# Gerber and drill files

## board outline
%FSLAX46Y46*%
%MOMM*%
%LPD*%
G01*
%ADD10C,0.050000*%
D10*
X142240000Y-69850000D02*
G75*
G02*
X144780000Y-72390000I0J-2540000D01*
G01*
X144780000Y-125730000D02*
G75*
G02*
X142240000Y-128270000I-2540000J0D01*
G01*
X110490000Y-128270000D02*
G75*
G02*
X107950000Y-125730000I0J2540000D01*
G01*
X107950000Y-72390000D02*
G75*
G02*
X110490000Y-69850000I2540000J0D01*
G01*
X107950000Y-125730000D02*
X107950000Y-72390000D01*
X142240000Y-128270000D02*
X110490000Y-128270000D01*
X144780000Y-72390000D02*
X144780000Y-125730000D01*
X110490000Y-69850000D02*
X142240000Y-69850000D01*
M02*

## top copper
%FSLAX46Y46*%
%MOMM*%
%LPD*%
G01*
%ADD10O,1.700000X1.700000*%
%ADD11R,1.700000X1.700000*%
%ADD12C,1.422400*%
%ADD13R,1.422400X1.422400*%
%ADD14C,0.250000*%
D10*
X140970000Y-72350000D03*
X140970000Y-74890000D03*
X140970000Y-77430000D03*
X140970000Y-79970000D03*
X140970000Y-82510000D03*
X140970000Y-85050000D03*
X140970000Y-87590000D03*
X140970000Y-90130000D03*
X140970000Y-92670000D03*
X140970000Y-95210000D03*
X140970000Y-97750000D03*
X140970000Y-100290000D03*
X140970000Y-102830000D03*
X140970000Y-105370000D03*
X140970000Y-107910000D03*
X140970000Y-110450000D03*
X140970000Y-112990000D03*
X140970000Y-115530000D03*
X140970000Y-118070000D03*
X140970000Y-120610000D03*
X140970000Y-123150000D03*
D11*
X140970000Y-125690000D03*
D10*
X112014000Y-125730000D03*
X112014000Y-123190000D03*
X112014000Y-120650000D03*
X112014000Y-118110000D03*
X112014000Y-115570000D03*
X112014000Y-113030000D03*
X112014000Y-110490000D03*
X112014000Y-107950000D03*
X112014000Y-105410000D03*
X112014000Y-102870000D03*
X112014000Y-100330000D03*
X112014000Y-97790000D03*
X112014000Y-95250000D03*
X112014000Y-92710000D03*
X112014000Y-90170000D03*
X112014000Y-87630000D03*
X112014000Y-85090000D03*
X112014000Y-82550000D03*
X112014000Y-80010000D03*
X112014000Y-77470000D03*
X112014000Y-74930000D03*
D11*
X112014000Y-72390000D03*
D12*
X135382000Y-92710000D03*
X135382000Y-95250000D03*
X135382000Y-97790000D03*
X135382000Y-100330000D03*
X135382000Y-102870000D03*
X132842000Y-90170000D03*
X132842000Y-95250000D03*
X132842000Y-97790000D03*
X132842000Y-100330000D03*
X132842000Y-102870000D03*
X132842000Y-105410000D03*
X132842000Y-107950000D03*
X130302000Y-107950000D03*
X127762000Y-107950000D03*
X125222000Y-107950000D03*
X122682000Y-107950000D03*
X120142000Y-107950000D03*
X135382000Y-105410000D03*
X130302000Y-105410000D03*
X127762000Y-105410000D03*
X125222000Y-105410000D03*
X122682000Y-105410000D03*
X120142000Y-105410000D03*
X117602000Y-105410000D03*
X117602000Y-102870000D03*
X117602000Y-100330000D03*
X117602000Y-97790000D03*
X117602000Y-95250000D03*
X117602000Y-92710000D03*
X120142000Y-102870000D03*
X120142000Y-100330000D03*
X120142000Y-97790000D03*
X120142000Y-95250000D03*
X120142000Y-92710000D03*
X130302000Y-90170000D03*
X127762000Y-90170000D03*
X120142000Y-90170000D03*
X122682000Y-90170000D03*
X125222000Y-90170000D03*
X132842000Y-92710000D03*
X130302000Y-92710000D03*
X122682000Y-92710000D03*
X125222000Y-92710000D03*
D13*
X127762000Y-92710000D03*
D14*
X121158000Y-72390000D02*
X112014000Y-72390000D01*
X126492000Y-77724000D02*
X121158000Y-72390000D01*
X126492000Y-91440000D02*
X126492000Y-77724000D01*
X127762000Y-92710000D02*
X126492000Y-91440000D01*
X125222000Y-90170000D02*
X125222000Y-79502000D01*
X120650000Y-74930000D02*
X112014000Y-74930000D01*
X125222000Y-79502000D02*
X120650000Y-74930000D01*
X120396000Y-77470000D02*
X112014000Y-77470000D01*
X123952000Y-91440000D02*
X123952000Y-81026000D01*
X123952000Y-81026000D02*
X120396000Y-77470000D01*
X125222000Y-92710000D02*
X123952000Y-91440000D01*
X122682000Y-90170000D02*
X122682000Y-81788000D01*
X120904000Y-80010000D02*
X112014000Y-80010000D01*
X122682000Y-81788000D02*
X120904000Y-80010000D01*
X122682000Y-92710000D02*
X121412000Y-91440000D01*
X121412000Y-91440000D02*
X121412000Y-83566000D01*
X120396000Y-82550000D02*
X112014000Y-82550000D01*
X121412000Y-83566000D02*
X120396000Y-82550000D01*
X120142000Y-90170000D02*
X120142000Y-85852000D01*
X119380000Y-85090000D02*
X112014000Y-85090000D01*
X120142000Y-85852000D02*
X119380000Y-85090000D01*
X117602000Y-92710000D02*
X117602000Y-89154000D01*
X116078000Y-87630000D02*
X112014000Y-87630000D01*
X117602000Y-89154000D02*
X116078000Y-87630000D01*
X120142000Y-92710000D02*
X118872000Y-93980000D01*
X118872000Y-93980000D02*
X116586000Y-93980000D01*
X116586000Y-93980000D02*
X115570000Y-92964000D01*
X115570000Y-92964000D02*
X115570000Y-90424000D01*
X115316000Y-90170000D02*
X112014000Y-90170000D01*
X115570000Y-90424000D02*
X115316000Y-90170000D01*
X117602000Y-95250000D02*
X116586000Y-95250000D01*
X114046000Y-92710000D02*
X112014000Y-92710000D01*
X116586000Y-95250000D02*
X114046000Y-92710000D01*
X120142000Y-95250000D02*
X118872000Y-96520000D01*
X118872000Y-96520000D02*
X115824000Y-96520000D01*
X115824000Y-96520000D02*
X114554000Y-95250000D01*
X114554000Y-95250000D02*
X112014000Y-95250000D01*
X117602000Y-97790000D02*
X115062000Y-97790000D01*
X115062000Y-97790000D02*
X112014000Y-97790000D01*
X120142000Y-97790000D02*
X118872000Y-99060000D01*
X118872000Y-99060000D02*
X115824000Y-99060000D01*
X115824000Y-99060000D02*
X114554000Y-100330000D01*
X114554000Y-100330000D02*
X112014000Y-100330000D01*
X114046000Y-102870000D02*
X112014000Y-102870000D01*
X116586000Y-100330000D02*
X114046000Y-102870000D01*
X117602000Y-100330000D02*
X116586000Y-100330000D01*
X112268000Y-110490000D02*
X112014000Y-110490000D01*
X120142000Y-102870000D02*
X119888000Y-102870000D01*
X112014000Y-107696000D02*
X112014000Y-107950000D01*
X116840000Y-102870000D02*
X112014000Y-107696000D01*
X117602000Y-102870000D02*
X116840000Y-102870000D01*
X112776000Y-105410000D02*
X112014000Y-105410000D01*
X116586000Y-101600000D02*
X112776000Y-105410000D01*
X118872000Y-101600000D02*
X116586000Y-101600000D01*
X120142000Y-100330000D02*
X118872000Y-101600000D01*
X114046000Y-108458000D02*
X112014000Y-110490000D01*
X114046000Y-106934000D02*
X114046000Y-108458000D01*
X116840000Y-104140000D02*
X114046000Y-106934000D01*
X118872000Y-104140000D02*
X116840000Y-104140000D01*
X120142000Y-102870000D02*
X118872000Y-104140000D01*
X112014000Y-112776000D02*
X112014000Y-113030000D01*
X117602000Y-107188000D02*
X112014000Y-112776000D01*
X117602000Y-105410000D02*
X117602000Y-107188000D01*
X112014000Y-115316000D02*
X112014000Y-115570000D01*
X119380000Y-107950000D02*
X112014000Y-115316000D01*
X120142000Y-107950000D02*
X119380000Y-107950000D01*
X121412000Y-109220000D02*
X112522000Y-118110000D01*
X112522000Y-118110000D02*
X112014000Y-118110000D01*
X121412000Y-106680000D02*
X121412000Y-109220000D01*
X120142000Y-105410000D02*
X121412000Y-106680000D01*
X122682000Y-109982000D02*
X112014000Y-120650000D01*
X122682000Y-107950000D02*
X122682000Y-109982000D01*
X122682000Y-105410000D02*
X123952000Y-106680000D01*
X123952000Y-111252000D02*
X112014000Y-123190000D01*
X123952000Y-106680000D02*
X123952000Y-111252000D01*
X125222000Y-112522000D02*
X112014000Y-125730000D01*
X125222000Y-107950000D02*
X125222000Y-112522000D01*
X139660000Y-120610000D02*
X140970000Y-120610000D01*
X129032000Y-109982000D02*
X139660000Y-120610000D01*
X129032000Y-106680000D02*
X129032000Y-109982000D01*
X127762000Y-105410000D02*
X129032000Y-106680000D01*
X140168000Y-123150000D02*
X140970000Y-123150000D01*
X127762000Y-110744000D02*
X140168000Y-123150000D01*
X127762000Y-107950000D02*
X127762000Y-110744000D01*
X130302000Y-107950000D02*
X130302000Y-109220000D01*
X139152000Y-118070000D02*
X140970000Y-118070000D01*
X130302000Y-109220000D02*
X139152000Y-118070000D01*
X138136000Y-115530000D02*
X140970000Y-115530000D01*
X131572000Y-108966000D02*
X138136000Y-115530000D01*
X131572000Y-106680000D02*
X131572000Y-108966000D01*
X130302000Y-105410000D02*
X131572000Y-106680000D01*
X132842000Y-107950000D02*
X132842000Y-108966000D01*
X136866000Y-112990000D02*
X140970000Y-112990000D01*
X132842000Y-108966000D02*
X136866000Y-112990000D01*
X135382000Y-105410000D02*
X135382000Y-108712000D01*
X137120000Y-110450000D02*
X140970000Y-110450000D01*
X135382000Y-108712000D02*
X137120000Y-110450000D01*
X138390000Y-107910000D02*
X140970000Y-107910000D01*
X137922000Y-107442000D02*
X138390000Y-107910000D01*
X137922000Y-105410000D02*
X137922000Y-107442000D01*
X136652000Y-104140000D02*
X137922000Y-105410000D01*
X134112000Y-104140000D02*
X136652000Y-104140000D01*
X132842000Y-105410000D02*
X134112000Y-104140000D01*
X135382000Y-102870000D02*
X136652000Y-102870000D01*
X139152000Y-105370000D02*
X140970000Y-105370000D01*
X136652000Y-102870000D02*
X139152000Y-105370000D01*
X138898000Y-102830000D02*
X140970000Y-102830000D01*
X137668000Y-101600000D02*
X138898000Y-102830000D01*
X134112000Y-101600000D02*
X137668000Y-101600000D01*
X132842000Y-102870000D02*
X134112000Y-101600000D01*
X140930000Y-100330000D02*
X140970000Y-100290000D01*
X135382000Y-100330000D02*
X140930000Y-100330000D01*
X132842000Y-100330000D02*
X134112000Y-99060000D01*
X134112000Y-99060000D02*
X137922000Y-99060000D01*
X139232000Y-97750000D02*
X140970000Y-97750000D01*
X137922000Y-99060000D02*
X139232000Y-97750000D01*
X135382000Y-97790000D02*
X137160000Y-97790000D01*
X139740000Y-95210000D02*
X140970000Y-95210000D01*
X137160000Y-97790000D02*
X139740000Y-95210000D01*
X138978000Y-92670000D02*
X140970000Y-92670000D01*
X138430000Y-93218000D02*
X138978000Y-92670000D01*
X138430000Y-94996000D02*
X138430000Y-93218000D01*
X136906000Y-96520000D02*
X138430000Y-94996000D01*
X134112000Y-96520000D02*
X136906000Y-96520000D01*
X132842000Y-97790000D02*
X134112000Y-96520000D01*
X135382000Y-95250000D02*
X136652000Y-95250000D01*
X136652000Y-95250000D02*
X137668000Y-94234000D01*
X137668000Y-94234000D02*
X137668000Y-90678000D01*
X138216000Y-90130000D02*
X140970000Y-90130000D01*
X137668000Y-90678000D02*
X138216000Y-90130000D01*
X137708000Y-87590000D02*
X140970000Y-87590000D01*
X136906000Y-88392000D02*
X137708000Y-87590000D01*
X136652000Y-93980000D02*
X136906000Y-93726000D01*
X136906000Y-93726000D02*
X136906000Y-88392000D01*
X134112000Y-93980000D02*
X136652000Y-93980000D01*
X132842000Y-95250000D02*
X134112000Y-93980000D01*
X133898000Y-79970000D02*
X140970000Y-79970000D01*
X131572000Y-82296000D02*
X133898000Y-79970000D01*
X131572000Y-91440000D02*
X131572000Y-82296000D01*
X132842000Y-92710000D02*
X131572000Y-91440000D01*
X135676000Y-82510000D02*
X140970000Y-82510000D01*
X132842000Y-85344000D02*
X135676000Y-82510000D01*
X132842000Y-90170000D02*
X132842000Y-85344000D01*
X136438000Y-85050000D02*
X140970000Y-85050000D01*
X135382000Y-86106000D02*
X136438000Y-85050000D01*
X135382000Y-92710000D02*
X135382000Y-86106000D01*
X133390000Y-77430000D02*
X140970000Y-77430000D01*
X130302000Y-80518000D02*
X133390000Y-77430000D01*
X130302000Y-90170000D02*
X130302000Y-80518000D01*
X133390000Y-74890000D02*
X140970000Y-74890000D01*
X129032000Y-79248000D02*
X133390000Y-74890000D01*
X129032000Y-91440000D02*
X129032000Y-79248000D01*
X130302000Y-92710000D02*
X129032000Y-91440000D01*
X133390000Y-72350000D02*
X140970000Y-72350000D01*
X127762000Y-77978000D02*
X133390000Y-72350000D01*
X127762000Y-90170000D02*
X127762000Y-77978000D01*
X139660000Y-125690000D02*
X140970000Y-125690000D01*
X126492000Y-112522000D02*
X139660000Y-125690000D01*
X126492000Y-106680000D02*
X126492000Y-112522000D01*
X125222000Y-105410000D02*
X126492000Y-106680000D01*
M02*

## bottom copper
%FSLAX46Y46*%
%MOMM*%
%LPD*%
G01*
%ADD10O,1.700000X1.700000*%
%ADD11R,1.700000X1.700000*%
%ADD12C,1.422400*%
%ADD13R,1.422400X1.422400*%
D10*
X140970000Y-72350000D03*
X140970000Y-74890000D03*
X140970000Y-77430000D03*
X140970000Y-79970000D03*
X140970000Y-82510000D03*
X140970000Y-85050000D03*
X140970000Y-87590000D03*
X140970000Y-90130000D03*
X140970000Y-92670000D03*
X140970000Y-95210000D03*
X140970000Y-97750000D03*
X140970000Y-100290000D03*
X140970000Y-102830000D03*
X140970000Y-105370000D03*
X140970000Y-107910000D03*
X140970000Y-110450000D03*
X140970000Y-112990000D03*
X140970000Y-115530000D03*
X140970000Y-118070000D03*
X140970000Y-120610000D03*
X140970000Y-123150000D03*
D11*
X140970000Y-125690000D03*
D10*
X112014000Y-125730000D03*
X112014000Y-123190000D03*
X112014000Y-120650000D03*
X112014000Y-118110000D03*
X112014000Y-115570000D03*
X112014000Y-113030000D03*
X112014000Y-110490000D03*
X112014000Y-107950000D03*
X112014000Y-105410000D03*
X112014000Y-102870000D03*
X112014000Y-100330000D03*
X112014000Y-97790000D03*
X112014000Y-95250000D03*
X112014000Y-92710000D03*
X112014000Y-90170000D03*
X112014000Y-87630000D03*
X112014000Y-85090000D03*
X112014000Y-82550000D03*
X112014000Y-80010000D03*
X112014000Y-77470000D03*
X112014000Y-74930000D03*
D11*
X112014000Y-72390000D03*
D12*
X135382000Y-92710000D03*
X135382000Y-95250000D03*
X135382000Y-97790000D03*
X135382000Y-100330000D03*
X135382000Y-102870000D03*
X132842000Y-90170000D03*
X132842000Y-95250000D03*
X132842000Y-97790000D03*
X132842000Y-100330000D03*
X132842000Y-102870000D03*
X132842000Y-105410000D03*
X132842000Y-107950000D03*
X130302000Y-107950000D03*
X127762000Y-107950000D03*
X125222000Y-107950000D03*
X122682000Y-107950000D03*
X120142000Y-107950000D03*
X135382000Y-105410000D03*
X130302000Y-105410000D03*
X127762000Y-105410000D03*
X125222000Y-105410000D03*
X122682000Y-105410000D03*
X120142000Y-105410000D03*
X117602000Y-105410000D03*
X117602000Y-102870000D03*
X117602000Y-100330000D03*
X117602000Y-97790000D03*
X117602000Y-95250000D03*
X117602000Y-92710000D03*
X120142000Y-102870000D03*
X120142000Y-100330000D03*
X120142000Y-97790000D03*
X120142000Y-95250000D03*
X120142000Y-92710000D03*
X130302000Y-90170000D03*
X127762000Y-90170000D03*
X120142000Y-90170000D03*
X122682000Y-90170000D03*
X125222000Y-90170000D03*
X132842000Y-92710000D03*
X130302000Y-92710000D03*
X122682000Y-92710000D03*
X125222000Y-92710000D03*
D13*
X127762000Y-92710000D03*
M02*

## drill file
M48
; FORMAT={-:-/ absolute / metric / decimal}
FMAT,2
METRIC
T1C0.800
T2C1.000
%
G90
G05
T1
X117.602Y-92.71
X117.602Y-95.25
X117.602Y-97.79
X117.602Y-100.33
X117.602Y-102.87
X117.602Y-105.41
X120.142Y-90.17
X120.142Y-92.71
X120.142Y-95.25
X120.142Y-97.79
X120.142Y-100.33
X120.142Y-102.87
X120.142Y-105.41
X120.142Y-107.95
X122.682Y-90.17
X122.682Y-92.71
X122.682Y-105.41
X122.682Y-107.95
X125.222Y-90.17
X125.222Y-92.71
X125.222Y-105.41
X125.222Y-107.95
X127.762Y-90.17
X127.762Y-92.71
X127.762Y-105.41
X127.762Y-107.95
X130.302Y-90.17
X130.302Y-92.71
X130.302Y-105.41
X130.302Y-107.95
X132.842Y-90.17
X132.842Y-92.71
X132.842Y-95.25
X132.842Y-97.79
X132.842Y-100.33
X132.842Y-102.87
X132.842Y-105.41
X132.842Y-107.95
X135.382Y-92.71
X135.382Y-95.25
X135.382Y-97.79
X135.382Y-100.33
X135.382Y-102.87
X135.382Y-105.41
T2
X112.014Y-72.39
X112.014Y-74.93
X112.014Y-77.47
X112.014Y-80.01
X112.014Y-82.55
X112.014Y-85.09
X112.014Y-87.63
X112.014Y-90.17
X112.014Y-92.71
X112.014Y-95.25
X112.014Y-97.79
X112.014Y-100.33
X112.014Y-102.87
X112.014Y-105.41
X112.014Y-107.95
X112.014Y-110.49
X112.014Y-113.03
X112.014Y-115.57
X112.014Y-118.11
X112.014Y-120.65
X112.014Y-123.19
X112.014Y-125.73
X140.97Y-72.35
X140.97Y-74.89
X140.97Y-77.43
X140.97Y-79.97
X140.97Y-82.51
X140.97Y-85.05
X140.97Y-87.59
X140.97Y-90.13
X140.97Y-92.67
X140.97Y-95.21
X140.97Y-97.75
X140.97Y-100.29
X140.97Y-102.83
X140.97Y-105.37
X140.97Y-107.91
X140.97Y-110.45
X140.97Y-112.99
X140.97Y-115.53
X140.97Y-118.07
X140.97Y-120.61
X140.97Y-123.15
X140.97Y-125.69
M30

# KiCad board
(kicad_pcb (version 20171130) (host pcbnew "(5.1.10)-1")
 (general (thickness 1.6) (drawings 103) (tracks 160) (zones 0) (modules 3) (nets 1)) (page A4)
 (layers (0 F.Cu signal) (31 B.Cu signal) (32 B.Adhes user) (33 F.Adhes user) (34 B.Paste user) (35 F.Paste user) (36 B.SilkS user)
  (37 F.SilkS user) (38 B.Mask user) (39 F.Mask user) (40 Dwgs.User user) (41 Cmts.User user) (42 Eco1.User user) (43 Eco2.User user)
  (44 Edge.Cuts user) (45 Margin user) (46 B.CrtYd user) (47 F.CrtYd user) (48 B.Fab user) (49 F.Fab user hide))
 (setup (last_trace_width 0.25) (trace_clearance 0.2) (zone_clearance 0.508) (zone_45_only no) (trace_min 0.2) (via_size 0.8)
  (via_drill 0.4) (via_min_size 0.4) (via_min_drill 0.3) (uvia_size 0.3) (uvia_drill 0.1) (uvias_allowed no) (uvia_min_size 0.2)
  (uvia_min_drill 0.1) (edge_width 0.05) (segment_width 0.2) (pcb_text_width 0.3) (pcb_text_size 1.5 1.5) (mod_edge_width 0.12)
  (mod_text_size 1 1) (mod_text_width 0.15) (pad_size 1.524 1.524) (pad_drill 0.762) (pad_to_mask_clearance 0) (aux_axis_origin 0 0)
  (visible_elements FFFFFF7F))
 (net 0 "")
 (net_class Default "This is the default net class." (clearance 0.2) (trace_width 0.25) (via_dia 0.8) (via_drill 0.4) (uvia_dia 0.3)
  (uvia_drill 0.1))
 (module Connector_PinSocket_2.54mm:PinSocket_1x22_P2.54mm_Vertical (layer F.Cu) (at 140.97 125.69 180)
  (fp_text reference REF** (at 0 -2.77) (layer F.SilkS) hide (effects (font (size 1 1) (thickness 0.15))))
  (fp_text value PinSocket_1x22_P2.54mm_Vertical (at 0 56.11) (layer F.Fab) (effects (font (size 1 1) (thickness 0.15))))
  (pad 22 thru_hole oval (at 0 53.34 180) (size 1.7 1.7) (drill 1) (layers *.Cu *.Mask))
  (pad 21 thru_hole oval (at 0 50.8 180) (size 1.7 1.7) (drill 1) (layers *.Cu *.Mask))
  (pad 20 thru_hole oval (at 0 48.26 180) (size 1.7 1.7) (drill 1) (layers *.Cu *.Mask))
  (pad 19 thru_hole oval (at 0 45.72 180) (size 1.7 1.7) (drill 1) (layers *.Cu *.Mask))
  (pad 18 thru_hole oval (at 0 43.18 180) (size 1.7 1.7) (drill 1) (layers *.Cu *.Mask))
  (pad 17 thru_hole oval (at 0 40.64 180) (size 1.7 1.7) (drill 1) (layers *.Cu *.Mask))
  (pad 16 thru_hole oval (at 0 38.1 180) (size 1.7 1.7) (drill 1) (layers *.Cu *.Mask))
  (pad 15 thru_hole oval (at 0 35.56 180) (size 1.7 1.7) (drill 1) (layers *.Cu *.Mask))
  (pad 14 thru_hole oval (at 0 33.02 180) (size 1.7 1.7) (drill 1) (layers *.Cu *.Mask))
  (pad 13 thru_hole oval (at 0 30.48 180) (size 1.7 1.7) (drill 1) (layers *.Cu *.Mask))
  (pad 12 thru_hole oval (at 0 27.94 180) (size 1.7 1.7) (drill 1) (layers *.Cu *.Mask))
  (pad 11 thru_hole oval (at 0 25.4 180) (size 1.7 1.7) (drill 1) (layers *.Cu *.Mask))
  (pad 10 thru_hole oval (at 0 22.86 180) (size 1.7 1.7) (drill 1) (layers *.Cu *.Mask))
  (pad 9 thru_hole oval (at 0 20.32 180) (size 1.7 1.7) (drill 1) (layers *.Cu *.Mask))
  (pad 8 thru_hole oval (at 0 17.78 180) (size 1.7 1.7) (drill 1) (layers *.Cu *.Mask))
  (pad 7 thru_hole oval (at 0 15.24 180) (size 1.7 1.7) (drill 1) (layers *.Cu *.Mask))
  (pad 6 thru_hole oval (at 0 12.7 180) (size 1.7 1.7) (drill 1) (layers *.Cu *.Mask))
  (pad 5 thru_hole oval (at 0 10.16 180) (size 1.7 1.7) (drill 1) (layers *.Cu *.Mask))
  (pad 4 thru_hole oval (at 0 7.62 180) (size 1.7 1.7) (drill 1) (layers *.Cu *.Mask))
  (pad 3 thru_hole oval (at 0 5.08 180) (size 1.7 1.7) (drill 1) (layers *.Cu *.Mask))
  (pad 2 thru_hole oval (at 0 2.54 180) (size 1.7 1.7) (drill 1) (layers *.Cu *.Mask))
  (pad 1 thru_hole rect (at 0 0 180) (size 1.7 1.7) (drill 1) (layers *.Cu *.Mask)))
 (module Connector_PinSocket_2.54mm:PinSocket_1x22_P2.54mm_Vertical (layer F.Cu) (at 112.014 72.39)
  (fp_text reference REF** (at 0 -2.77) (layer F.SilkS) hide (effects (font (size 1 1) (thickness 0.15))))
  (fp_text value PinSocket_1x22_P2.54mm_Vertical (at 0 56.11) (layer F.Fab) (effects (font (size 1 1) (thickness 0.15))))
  (pad 22 thru_hole oval (at 0 53.34) (size 1.7 1.7) (drill 1) (layers *.Cu *.Mask))
  (pad 21 thru_hole oval (at 0 50.8) (size 1.7 1.7) (drill 1) (layers *.Cu *.Mask))
  (pad 20 thru_hole oval (at 0 48.26) (size 1.7 1.7) (drill 1) (layers *.Cu *.Mask))
  (pad 19 thru_hole oval (at 0 45.72) (size 1.7 1.7) (drill 1) (layers *.Cu *.Mask))
  (pad 18 thru_hole oval (at 0 43.18) (size 1.7 1.7) (drill 1) (layers *.Cu *.Mask))
  (pad 17 thru_hole oval (at 0 40.64) (size 1.7 1.7) (drill 1) (layers *.Cu *.Mask))
  (pad 16 thru_hole oval (at 0 38.1) (size 1.7 1.7) (drill 1) (layers *.Cu *.Mask))
  (pad 15 thru_hole oval (at 0 35.56) (size 1.7 1.7) (drill 1) (layers *.Cu *.Mask))
  (pad 14 thru_hole oval (at 0 33.02) (size 1.7 1.7) (drill 1) (layers *.Cu *.Mask))
  (pad 13 thru_hole oval (at 0 30.48) (size 1.7 1.7) (drill 1) (layers *.Cu *.Mask))
  (pad 12 thru_hole oval (at 0 27.94) (size 1.7 1.7) (drill 1) (layers *.Cu *.Mask))
  (pad 11 thru_hole oval (at 0 25.4) (size 1.7 1.7) (drill 1) (layers *.Cu *.Mask))
  (pad 10 thru_hole oval (at 0 22.86) (size 1.7 1.7) (drill 1) (layers *.Cu *.Mask))
  (pad 9 thru_hole oval (at 0 20.32) (size 1.7 1.7) (drill 1) (layers *.Cu *.Mask))
  (pad 8 thru_hole oval (at 0 17.78) (size 1.7 1.7) (drill 1) (layers *.Cu *.Mask))
  (pad 7 thru_hole oval (at 0 15.24) (size 1.7 1.7) (drill 1) (layers *.Cu *.Mask))
  (pad 6 thru_hole oval (at 0 12.7) (size 1.7 1.7) (drill 1) (layers *.Cu *.Mask))
  (pad 5 thru_hole oval (at 0 10.16) (size 1.7 1.7) (drill 1) (layers *.Cu *.Mask))
  (pad 4 thru_hole oval (at 0 7.62) (size 1.7 1.7) (drill 1) (layers *.Cu *.Mask))
  (pad 3 thru_hole oval (at 0 5.08) (size 1.7 1.7) (drill 1) (layers *.Cu *.Mask))
  (pad 2 thru_hole oval (at 0 2.54) (size 1.7 1.7) (drill 1) (layers *.Cu *.Mask))
  (pad 1 thru_hole rect (at 0 0) (size 1.7 1.7) (drill 1) (layers *.Cu *.Mask)))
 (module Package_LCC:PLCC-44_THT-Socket (layer F.Cu) (at 127.762 92.71)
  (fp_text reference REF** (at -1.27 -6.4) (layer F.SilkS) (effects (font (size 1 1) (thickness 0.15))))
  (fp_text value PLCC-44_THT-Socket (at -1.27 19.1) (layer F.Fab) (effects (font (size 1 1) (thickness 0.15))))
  (pad 39 thru_hole circle (at 7.62 0) (size 1.4224 1.4224) (drill 0.8) (layers *.Cu *.Mask))
  (pad 37 thru_hole circle (at 7.62 2.54) (size 1.4224 1.4224) (drill 0.8) (layers *.Cu *.Mask))
  (pad 35 thru_hole circle (at 7.62 5.08) (size 1.4224 1.4224) (drill 0.8) (layers *.Cu *.Mask))
  (pad 33 thru_hole circle (at 7.62 7.62) (size 1.4224 1.4224) (drill 0.8) (layers *.Cu *.Mask))
  (pad 31 thru_hole circle (at 7.62 10.16) (size 1.4224 1.4224) (drill 0.8) (layers *.Cu *.Mask))
  (pad 40 thru_hole circle (at 5.08 -2.54) (size 1.4224 1.4224) (drill 0.8) (layers *.Cu *.Mask))
  (pad 38 thru_hole circle (at 5.08 2.54) (size 1.4224 1.4224) (drill 0.8) (layers *.Cu *.Mask))
  (pad 36 thru_hole circle (at 5.08 5.08) (size 1.4224 1.4224) (drill 0.8) (layers *.Cu *.Mask))
  (pad 34 thru_hole circle (at 5.08 7.62) (size 1.4224 1.4224) (drill 0.8) (layers *.Cu *.Mask))
  (pad 32 thru_hole circle (at 5.08 10.16) (size 1.4224 1.4224) (drill 0.8) (layers *.Cu *.Mask))
  (pad 30 thru_hole circle (at 5.08 12.7) (size 1.4224 1.4224) (drill 0.8) (layers *.Cu *.Mask))
  (pad 28 thru_hole circle (at 5.08 15.24) (size 1.4224 1.4224) (drill 0.8) (layers *.Cu *.Mask))
  (pad 26 thru_hole circle (at 2.54 15.24) (size 1.4224 1.4224) (drill 0.8) (layers *.Cu *.Mask))
  (pad 24 thru_hole circle (at 0 15.24) (size 1.4224 1.4224) (drill 0.8) (layers *.Cu *.Mask))
  (pad 22 thru_hole circle (at -2.54 15.24) (size 1.4224 1.4224) (drill 0.8) (layers *.Cu *.Mask))
  (pad 20 thru_hole circle (at -5.08 15.24) (size 1.4224 1.4224) (drill 0.8) (layers *.Cu *.Mask))
  (pad 18 thru_hole circle (at -7.62 15.24) (size 1.4224 1.4224) (drill 0.8) (layers *.Cu *.Mask))
  (pad 29 thru_hole circle (at 7.62 12.7) (size 1.4224 1.4224) (drill 0.8) (layers *.Cu *.Mask))
  (pad 27 thru_hole circle (at 2.54 12.7) (size 1.4224 1.4224) (drill 0.8) (layers *.Cu *.Mask))
  (pad 25 thru_hole circle (at 0 12.7) (size 1.4224 1.4224) (drill 0.8) (layers *.Cu *.Mask))
  (pad 23 thru_hole circle (at -2.54 12.7) (size 1.4224 1.4224) (drill 0.8) (layers *.Cu *.Mask))
  (pad 21 thru_hole circle (at -5.08 12.7) (size 1.4224 1.4224) (drill 0.8) (layers *.Cu *.Mask))
  (pad 19 thru_hole circle (at -7.62 12.7) (size 1.4224 1.4224) (drill 0.8) (layers *.Cu *.Mask))
  (pad 17 thru_hole circle (at -10.16 12.7) (size 1.4224 1.4224) (drill 0.8) (layers *.Cu *.Mask))
  (pad 15 thru_hole circle (at -10.16 10.16) (size 1.4224 1.4224) (drill 0.8) (layers *.Cu *.Mask))
  (pad 13 thru_hole circle (at -10.16 7.62) (size 1.4224 1.4224) (drill 0.8) (layers *.Cu *.Mask))
  (pad 11 thru_hole circle (at -10.16 5.08) (size 1.4224 1.4224) (drill 0.8) (layers *.Cu *.Mask))
  (pad 9 thru_hole circle (at -10.16 2.54) (size 1.4224 1.4224) (drill 0.8) (layers *.Cu *.Mask))
  (pad 7 thru_hole circle (at -10.16 0) (size 1.4224 1.4224) (drill 0.8) (layers *.Cu *.Mask))
  (pad 16 thru_hole circle (at -7.62 10.16) (size 1.4224 1.4224) (drill 0.8) (layers *.Cu *.Mask))
  (pad 14 thru_hole circle (at -7.62 7.62) (size 1.4224 1.4224) (drill 0.8) (layers *.Cu *.Mask))
  (pad 12 thru_hole circle (at -7.62 5.08) (size 1.4224 1.4224) (drill 0.8) (layers *.Cu *.Mask))
  (pad 10 thru_hole circle (at -7.62 2.54) (size 1.4224 1.4224) (drill 0.8) (layers *.Cu *.Mask))
  (pad 8 thru_hole circle (at -7.62 0) (size 1.4224 1.4224) (drill 0.8) (layers *.Cu *.Mask))
  (pad 42 thru_hole circle (at 2.54 -2.54) (size 1.4224 1.4224) (drill 0.8) (layers *.Cu *.Mask))
  (pad 44 thru_hole circle (at 0 -2.54) (size 1.4224 1.4224) (drill 0.8) (layers *.Cu *.Mask))
  (pad 6 thru_hole circle (at -7.62 -2.54) (size 1.4224 1.4224) (drill 0.8) (layers *.Cu *.Mask))
  (pad 4 thru_hole circle (at -5.08 -2.54) (size 1.4224 1.4224) (drill 0.8) (layers *.Cu *.Mask))
  (pad 2 thru_hole circle (at -2.54 -2.54) (size 1.4224 1.4224) (drill 0.8) (layers *.Cu *.Mask))
  (pad 41 thru_hole circle (at 5.08 0) (size 1.4224 1.4224) (drill 0.8) (layers *.Cu *.Mask))
  (pad 43 thru_hole circle (at 2.54 0) (size 1.4224 1.4224) (drill 0.8) (layers *.Cu *.Mask))
  (pad 5 thru_hole circle (at -5.08 0) (size 1.4224 1.4224) (drill 0.8) (layers *.Cu *.Mask))
  (pad 3 thru_hole circle (at -2.54 0) (size 1.4224 1.4224) (drill 0.8) (layers *.Cu *.Mask))
  (pad 1 thru_hole rect (at 0 0) (size 1.4224 1.4224) (drill 0.8) (layers *.Cu *.Mask)))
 (gr_arc (start 142.24 72.39) (end 144.78 72.39) (angle -90) (layer Edge.Cuts) (width 0.05))
 (gr_arc (start 142.24 125.73) (end 142.24 128.27) (angle -90) (layer Edge.Cuts) (width 0.05))
 (gr_arc (start 110.49 125.73) (end 107.95 125.73) (angle -90) (layer Edge.Cuts) (width 0.05))
 (gr_arc (start 110.49 72.39) (end 110.49 69.85) (angle -90) (layer Edge.Cuts) (width 0.05))
 (gr_line (start 107.95 125.73) (end 107.95 72.39) (layer Edge.Cuts) (width 0.05))
 (gr_line (start 142.24 128.27) (end 110.49 128.27) (layer Edge.Cuts) (width 0.05))
 (gr_line (start 144.78 72.39) (end 144.78 125.73) (layer Edge.Cuts) (width 0.05))
 (gr_line (start 110.49 69.85) (end 142.24 69.85) (layer Edge.Cuts) (width 0.05))
 (segment (start 121.158 72.39) (end 112.014 72.39) (width 0.25) (layer F.Cu) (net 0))
 (segment (start 126.492 77.724) (end 121.158 72.39) (width 0.25) (layer F.Cu) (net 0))
 (segment (start 126.492 91.44) (end 126.492 77.724) (width 0.25) (layer F.Cu) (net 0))
 (segment (start 127.762 92.71) (end 126.492 91.44) (width 0.25) (layer F.Cu) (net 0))
 (segment (start 125.222 90.17) (end 125.222 79.502) (width 0.25) (layer F.Cu) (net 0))
 (segment (start 120.65 74.93) (end 112.014 74.93) (width 0.25) (layer F.Cu) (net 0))
 (segment (start 125.222 79.502) (end 120.65 74.93) (width 0.25) (layer F.Cu) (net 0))
 (segment (start 120.396 77.47) (end 112.014 77.47) (width 0.25) (layer F.Cu) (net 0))
 (segment (start 123.952 91.44) (end 123.952 81.026) (width 0.25) (layer F.Cu) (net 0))
 (segment (start 123.952 81.026) (end 120.396 77.47) (width 0.25) (layer F.Cu) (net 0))
 (segment (start 125.222 92.71) (end 123.952 91.44) (width 0.25) (layer F.Cu) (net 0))
 (segment (start 122.682 90.17) (end 122.682 81.788) (width 0.25) (layer F.Cu) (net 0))
 (segment (start 120.904 80.01) (end 112.014 80.01) (width 0.25) (layer F.Cu) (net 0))
 (segment (start 122.682 81.788) (end 120.904 80.01) (width 0.25) (layer F.Cu) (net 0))
 (segment (start 122.682 92.71) (end 121.412 91.44) (width 0.25) (layer F.Cu) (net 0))
 (segment (start 121.412 91.44) (end 121.412 83.566) (width 0.25) (layer F.Cu) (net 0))
 (segment (start 120.396 82.55) (end 112.014 82.55) (width 0.25) (layer F.Cu) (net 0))
 (segment (start 121.412 83.566) (end 120.396 82.55) (width 0.25) (layer F.Cu) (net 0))
 (segment (start 120.142 90.17) (end 120.142 85.852) (width 0.25) (layer F.Cu) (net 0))
 (segment (start 119.38 85.09) (end 112.014 85.09) (width 0.25) (layer F.Cu) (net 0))
 (segment (start 120.142 85.852) (end 119.38 85.09) (width 0.25) (layer F.Cu) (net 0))
 (segment (start 117.602 92.71) (end 117.602 89.154) (width 0.25) (layer F.Cu) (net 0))
 (segment (start 116.078 87.63) (end 112.014 87.63) (width 0.25) (layer F.Cu) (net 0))
 (segment (start 117.602 89.154) (end 116.078 87.63) (width 0.25) (layer F.Cu) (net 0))
 (segment (start 120.142 92.71) (end 118.872 93.98) (width 0.25) (layer F.Cu) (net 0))
 (segment (start 118.872 93.98) (end 116.586 93.98) (width 0.25) (layer F.Cu) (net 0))
 (segment (start 116.586 93.98) (end 115.57 92.964) (width 0.25) (layer F.Cu) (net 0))
 (segment (start 115.57 92.964) (end 115.57 90.424) (width 0.25) (layer F.Cu) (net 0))
 (segment (start 115.316 90.17) (end 112.014 90.17) (width 0.25) (layer F.Cu) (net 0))
 (segment (start 115.57 90.424) (end 115.316 90.17) (width 0.25) (layer F.Cu) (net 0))
 (segment (start 117.602 95.25) (end 116.586 95.25) (width 0.25) (layer F.Cu) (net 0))
 (segment (start 114.046 92.71) (end 112.014 92.71) (width 0.25) (layer F.Cu) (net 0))
 (segment (start 116.586 95.25) (end 114.046 92.71) (width 0.25) (layer F.Cu) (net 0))
 (segment (start 120.142 95.25) (end 118.872 96.52) (width 0.25) (layer F.Cu) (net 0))
 (segment (start 118.872 96.52) (end 115.824 96.52) (width 0.25) (layer F.Cu) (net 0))
 (segment (start 115.824 96.52) (end 114.554 95.25) (width 0.25) (layer F.Cu) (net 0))
 (segment (start 114.554 95.25) (end 112.014 95.25) (width 0.25) (layer F.Cu) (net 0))
 (segment (start 117.602 97.79) (end 115.062 97.79) (width 0.25) (layer F.Cu) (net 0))
 (segment (start 115.062 97.79) (end 112.014 97.79) (width 0.25) (layer F.Cu) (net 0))
 (segment (start 120.142 97.79) (end 118.872 99.06) (width 0.25) (layer F.Cu) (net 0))
 (segment (start 118.872 99.06) (end 115.824 99.06) (width 0.25) (layer F.Cu) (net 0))
 (segment (start 115.824 99.06) (end 114.554 100.33) (width 0.25) (layer F.Cu) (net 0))
 (segment (start 114.554 100.33) (end 112.014 100.33) (width 0.25) (layer F.Cu) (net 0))
 (segment (start 114.046 102.87) (end 112.014 102.87) (width 0.25) (layer F.Cu) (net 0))
 (segment (start 116.586 100.33) (end 114.046 102.87) (width 0.25) (layer F.Cu) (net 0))
 (segment (start 117.602 100.33) (end 116.586 100.33) (width 0.25) (layer F.Cu) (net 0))
 (segment (start 112.268 110.49) (end 112.014 110.49) (width 0.25) (layer F.Cu) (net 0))
 (segment (start 120.142 102.87) (end 119.888 102.87) (width 0.25) (layer F.Cu) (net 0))
 (segment (start 112.014 107.696) (end 112.014 107.95) (width 0.25) (layer F.Cu) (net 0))
 (segment (start 116.84 102.87) (end 112.014 107.696) (width 0.25) (layer F.Cu) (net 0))
 (segment (start 117.602 102.87) (end 116.84 102.87) (width 0.25) (layer F.Cu) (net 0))
 (segment (start 112.776 105.41) (end 112.014 105.41) (width 0.25) (layer F.Cu) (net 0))
 (segment (start 116.586 101.6) (end 112.776 105.41) (width 0.25) (layer F.Cu) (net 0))
 (segment (start 118.872 101.6) (end 116.586 101.6) (width 0.25) (layer F.Cu) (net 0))
 (segment (start 120.142 100.33) (end 118.872 101.6) (width 0.25) (layer F.Cu) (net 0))
 (segment (start 114.046 108.458) (end 112.014 110.49) (width 0.25) (layer F.Cu) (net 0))
 (segment (start 114.046 106.934) (end 114.046 108.458) (width 0.25) (layer F.Cu) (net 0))
 (segment (start 116.84 104.14) (end 114.046 106.934) (width 0.25) (layer F.Cu) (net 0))
 (segment (start 118.872 104.14) (end 116.84 104.14) (width 0.25) (layer F.Cu) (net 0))
 (segment (start 120.142 102.87) (end 118.872 104.14) (width 0.25) (layer F.Cu) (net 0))
 (segment (start 112.014 112.776) (end 112.014 113.03) (width 0.25) (layer F.Cu) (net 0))
 (segment (start 117.602 107.188) (end 112.014 112.776) (width 0.25) (layer F.Cu) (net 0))
 (segment (start 117.602 105.41) (end 117.602 107.188) (width 0.25) (layer F.Cu) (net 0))
 (segment (start 112.014 115.316) (end 112.014 115.57) (width 0.25) (layer F.Cu) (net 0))
 (segment (start 119.38 107.95) (end 112.014 115.316) (width 0.25) (layer F.Cu) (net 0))
 (segment (start 120.142 107.95) (end 119.38 107.95) (width 0.25) (layer F.Cu) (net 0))
 (segment (start 121.412 109.22) (end 112.522 118.11) (width 0.25) (layer F.Cu) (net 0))
 (segment (start 112.522 118.11) (end 112.014 118.11) (width 0.25) (layer F.Cu) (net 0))
 (segment (start 121.412 106.68) (end 121.412 109.22) (width 0.25) (layer F.Cu) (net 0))
 (segment (start 120.142 105.41) (end 121.412 106.68) (width 0.25) (layer F.Cu) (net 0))
 (segment (start 122.682 109.982) (end 112.014 120.65) (width 0.25) (layer F.Cu) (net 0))
 (segment (start 122.682 107.95) (end 122.682 109.982) (width 0.25) (layer F.Cu) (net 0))
 (segment (start 122.682 105.41) (end 123.952 106.68) (width 0.25) (layer F.Cu) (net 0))
 (segment (start 123.952 111.252) (end 112.014 123.19) (width 0.25) (layer F.Cu) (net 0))
 (segment (start 123.952 106.68) (end 123.952 111.252) (width 0.25) (layer F.Cu) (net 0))
 (segment (start 125.222 112.522) (end 112.014 125.73) (width 0.25) (layer F.Cu) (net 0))
 (segment (start 125.222 107.95) (end 125.222 112.522) (width 0.25) (layer F.Cu) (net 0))
 (segment (start 139.66 120.61) (end 140.97 120.61) (width 0.25) (layer F.Cu) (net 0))
 (segment (start 129.032 109.982) (end 139.66 120.61) (width 0.25) (layer F.Cu) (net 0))
 (segment (start 129.032 106.68) (end 129.032 109.982) (width 0.25) (layer F.Cu) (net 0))
 (segment (start 127.762 105.41) (end 129.032 106.68) (width 0.25) (layer F.Cu) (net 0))
 (segment (start 140.168 123.15) (end 140.97 123.15) (width 0.25) (layer F.Cu) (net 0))
 (segment (start 127.762 110.744) (end 140.168 123.15) (width 0.25) (layer F.Cu) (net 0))
 (segment (start 127.762 107.95) (end 127.762 110.744) (width 0.25) (layer F.Cu) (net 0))
 (segment (start 130.302 107.95) (end 130.302 109.22) (width 0.25) (layer F.Cu) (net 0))
 (segment (start 139.152 118.07) (end 140.97 118.07) (width 0.25) (layer F.Cu) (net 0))
 (segment (start 130.302 109.22) (end 139.152 118.07) (width 0.25) (layer F.Cu) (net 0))
 (segment (start 138.136 115.53) (end 140.97 115.53) (width 0.25) (layer F.Cu) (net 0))
 (segment (start 131.572 108.966) (end 138.136 115.53) (width 0.25) (layer F.Cu) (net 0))
 (segment (start 131.572 106.68) (end 131.572 108.966) (width 0.25) (layer F.Cu) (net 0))
 (segment (start 130.302 105.41) (end 131.572 106.68) (width 0.25) (layer F.Cu) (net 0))
 (segment (start 132.842 107.95) (end 132.842 108.966) (width 0.25) (layer F.Cu) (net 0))
 (segment (start 136.866 112.99) (end 140.97 112.99) (width 0.25) (layer F.Cu) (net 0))
 (segment (start 132.842 108.966) (end 136.866 112.99) (width 0.25) (layer F.Cu) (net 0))
 (segment (start 135.382 105.41) (end 135.382 108.712) (width 0.25) (layer F.Cu) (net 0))
 (segment (start 137.12 110.45) (end 140.97 110.45) (width 0.25) (layer F.Cu) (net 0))
 (segment (start 135.382 108.712) (end 137.12 110.45) (width 0.25) (layer F.Cu) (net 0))
 (segment (start 138.39 107.91) (end 140.97 107.91) (width 0.25) (layer F.Cu) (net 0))
 (segment (start 137.922 107.442) (end 138.39 107.91) (width 0.25) (layer F.Cu) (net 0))
 (segment (start 137.922 105.41) (end 137.922 107.442) (width 0.25) (layer F.Cu) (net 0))
 (segment (start 136.652 104.14) (end 137.922 105.41) (width 0.25) (layer F.Cu) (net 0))
 (segment (start 134.112 104.14) (end 136.652 104.14) (width 0.25) (layer F.Cu) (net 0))
 (segment (start 132.842 105.41) (end 134.112 104.14) (width 0.25) (layer F.Cu) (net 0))
 (segment (start 135.382 102.87) (end 136.652 102.87) (width 0.25) (layer F.Cu) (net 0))
 (segment (start 139.152 105.37) (end 140.97 105.37) (width 0.25) (layer F.Cu) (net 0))
 (segment (start 136.652 102.87) (end 139.152 105.37) (width 0.25) (layer F.Cu) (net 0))
 (segment (start 138.898 102.83) (end 140.97 102.83) (width 0.25) (layer F.Cu) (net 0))
 (segment (start 137.668 101.6) (end 138.898 102.83) (width 0.25) (layer F.Cu) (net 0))
 (segment (start 134.112 101.6) (end 137.668 101.6) (width 0.25) (layer F.Cu) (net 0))
 (segment (start 132.842 102.87) (end 134.112 101.6) (width 0.25) (layer F.Cu) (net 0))
 (segment (start 140.93 100.33) (end 140.97 100.29) (width 0.25) (layer F.Cu) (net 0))
 (segment (start 135.382 100.33) (end 140.93 100.33) (width 0.25) (layer F.Cu) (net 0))
 (segment (start 132.842 100.33) (end 134.112 99.06) (width 0.25) (layer F.Cu) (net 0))
 (segment (start 134.112 99.06) (end 137.922 99.06) (width 0.25) (layer F.Cu) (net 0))
 (segment (start 139.232 97.75) (end 140.97 97.75) (width 0.25) (layer F.Cu) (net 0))
 (segment (start 137.922 99.06) (end 139.232 97.75) (width 0.25) (layer F.Cu) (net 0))
 (segment (start 135.382 97.79) (end 137.16 97.79) (width 0.25) (layer F.Cu) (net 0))
 (segment (start 139.74 95.21) (end 140.97 95.21) (width 0.25) (layer F.Cu) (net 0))
 (segment (start 137.16 97.79) (end 139.74 95.21) (width 0.25) (layer F.Cu) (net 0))
 (segment (start 138.978 92.67) (end 140.97 92.67) (width 0.25) (layer F.Cu) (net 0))
 (segment (start 138.43 93.218) (end 138.978 92.67) (width 0.25) (layer F.Cu) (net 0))
 (segment (start 138.43 94.996) (end 138.43 93.218) (width 0.25) (layer F.Cu) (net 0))
 (segment (start 136.906 96.52) (end 138.43 94.996) (width 0.25) (layer F.Cu) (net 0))
 (segment (start 134.112 96.52) (end 136.906 96.52) (width 0.25) (layer F.Cu) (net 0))
 (segment (start 132.842 97.79) (end 134.112 96.52) (width 0.25) (layer F.Cu) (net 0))
 (segment (start 135.382 95.25) (end 136.652 95.25) (width 0.25) (layer F.Cu) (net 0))
 (segment (start 136.652 95.25) (end 137.668 94.234) (width 0.25) (layer F.Cu) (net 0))
 (segment (start 137.668 94.234) (end 137.668 90.678) (width 0.25) (layer F.Cu) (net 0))
 (segment (start 138.216 90.13) (end 140.97 90.13) (width 0.25) (layer F.Cu) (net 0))
 (segment (start 137.668 90.678) (end 138.216 90.13) (width 0.25) (layer F.Cu) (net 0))
 (segment (start 137.708 87.59) (end 140.97 87.59) (width 0.25) (layer F.Cu) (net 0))
 (segment (start 136.906 88.392) (end 137.708 87.59) (width 0.25) (layer F.Cu) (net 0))
 (segment (start 136.652 93.98) (end 136.906 93.726) (width 0.25) (layer F.Cu) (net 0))
 (segment (start 136.906 93.726) (end 136.906 88.392) (width 0.25) (layer F.Cu) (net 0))
 (segment (start 134.112 93.98) (end 136.652 93.98) (width 0.25) (layer F.Cu) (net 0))
 (segment (start 132.842 95.25) (end 134.112 93.98) (width 0.25) (layer F.Cu) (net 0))
 (segment (start 133.898 79.97) (end 140.97 79.97) (width 0.25) (layer F.Cu) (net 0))
 (segment (start 131.572 82.296) (end 133.898 79.97) (width 0.25) (layer F.Cu) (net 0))
 (segment (start 131.572 91.44) (end 131.572 82.296) (width 0.25) (layer F.Cu) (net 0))
 (segment (start 132.842 92.71) (end 131.572 91.44) (width 0.25) (layer F.Cu) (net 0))
 (segment (start 135.676 82.51) (end 140.97 82.51) (width 0.25) (layer F.Cu) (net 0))
 (segment (start 132.842 85.344) (end 135.676 82.51) (width 0.25) (layer F.Cu) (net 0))
 (segment (start 132.842 90.17) (end 132.842 85.344) (width 0.25) (layer F.Cu) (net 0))
 (segment (start 136.438 85.05) (end 140.97 85.05) (width 0.25) (layer F.Cu) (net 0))
 (segment (start 135.382 86.106) (end 136.438 85.05) (width 0.25) (layer F.Cu) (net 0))
 (segment (start 135.382 92.71) (end 135.382 86.106) (width 0.25) (layer F.Cu) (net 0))
 (segment (start 133.39 77.43) (end 140.97 77.43) (width 0.25) (layer F.Cu) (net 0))
 (segment (start 130.302 80.518) (end 133.39 77.43) (width 0.25) (layer F.Cu) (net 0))
 (segment (start 130.302 90.17) (end 130.302 80.518) (width 0.25) (layer F.Cu) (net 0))
 (segment (start 133.39 74.89) (end 140.97 74.89) (width 0.25) (layer F.Cu) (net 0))
 (segment (start 129.032 79.248) (end 133.39 74.89) (width 0.25) (layer F.Cu) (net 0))
 (segment (start 129.032 91.44) (end 129.032 79.248) (width 0.25) (layer F.Cu) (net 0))
 (segment (start 130.302 92.71) (end 129.032 91.44) (width 0.25) (layer F.Cu) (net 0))
 (segment (start 133.39 72.35) (end 140.97 72.35) (width 0.25) (layer F.Cu) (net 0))
 (segment (start 127.762 77.978) (end 133.39 72.35) (width 0.25) (layer F.Cu) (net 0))
 (segment (start 127.762 90.17) (end 127.762 77.978) (width 0.25) (layer F.Cu) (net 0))
 (segment (start 139.66 125.69) (end 140.97 125.69) (width 0.25) (layer F.Cu) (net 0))
 (segment (start 126.492 112.522) (end 139.66 125.69) (width 0.25) (layer F.Cu) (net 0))
 (segment (start 126.492 106.68) (end 126.492 112.522) (width 0.25) (layer F.Cu) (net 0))
 (segment (start 125.222 105.41) (end 126.492 106.68) (width 0.25) (layer F.Cu) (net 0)))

